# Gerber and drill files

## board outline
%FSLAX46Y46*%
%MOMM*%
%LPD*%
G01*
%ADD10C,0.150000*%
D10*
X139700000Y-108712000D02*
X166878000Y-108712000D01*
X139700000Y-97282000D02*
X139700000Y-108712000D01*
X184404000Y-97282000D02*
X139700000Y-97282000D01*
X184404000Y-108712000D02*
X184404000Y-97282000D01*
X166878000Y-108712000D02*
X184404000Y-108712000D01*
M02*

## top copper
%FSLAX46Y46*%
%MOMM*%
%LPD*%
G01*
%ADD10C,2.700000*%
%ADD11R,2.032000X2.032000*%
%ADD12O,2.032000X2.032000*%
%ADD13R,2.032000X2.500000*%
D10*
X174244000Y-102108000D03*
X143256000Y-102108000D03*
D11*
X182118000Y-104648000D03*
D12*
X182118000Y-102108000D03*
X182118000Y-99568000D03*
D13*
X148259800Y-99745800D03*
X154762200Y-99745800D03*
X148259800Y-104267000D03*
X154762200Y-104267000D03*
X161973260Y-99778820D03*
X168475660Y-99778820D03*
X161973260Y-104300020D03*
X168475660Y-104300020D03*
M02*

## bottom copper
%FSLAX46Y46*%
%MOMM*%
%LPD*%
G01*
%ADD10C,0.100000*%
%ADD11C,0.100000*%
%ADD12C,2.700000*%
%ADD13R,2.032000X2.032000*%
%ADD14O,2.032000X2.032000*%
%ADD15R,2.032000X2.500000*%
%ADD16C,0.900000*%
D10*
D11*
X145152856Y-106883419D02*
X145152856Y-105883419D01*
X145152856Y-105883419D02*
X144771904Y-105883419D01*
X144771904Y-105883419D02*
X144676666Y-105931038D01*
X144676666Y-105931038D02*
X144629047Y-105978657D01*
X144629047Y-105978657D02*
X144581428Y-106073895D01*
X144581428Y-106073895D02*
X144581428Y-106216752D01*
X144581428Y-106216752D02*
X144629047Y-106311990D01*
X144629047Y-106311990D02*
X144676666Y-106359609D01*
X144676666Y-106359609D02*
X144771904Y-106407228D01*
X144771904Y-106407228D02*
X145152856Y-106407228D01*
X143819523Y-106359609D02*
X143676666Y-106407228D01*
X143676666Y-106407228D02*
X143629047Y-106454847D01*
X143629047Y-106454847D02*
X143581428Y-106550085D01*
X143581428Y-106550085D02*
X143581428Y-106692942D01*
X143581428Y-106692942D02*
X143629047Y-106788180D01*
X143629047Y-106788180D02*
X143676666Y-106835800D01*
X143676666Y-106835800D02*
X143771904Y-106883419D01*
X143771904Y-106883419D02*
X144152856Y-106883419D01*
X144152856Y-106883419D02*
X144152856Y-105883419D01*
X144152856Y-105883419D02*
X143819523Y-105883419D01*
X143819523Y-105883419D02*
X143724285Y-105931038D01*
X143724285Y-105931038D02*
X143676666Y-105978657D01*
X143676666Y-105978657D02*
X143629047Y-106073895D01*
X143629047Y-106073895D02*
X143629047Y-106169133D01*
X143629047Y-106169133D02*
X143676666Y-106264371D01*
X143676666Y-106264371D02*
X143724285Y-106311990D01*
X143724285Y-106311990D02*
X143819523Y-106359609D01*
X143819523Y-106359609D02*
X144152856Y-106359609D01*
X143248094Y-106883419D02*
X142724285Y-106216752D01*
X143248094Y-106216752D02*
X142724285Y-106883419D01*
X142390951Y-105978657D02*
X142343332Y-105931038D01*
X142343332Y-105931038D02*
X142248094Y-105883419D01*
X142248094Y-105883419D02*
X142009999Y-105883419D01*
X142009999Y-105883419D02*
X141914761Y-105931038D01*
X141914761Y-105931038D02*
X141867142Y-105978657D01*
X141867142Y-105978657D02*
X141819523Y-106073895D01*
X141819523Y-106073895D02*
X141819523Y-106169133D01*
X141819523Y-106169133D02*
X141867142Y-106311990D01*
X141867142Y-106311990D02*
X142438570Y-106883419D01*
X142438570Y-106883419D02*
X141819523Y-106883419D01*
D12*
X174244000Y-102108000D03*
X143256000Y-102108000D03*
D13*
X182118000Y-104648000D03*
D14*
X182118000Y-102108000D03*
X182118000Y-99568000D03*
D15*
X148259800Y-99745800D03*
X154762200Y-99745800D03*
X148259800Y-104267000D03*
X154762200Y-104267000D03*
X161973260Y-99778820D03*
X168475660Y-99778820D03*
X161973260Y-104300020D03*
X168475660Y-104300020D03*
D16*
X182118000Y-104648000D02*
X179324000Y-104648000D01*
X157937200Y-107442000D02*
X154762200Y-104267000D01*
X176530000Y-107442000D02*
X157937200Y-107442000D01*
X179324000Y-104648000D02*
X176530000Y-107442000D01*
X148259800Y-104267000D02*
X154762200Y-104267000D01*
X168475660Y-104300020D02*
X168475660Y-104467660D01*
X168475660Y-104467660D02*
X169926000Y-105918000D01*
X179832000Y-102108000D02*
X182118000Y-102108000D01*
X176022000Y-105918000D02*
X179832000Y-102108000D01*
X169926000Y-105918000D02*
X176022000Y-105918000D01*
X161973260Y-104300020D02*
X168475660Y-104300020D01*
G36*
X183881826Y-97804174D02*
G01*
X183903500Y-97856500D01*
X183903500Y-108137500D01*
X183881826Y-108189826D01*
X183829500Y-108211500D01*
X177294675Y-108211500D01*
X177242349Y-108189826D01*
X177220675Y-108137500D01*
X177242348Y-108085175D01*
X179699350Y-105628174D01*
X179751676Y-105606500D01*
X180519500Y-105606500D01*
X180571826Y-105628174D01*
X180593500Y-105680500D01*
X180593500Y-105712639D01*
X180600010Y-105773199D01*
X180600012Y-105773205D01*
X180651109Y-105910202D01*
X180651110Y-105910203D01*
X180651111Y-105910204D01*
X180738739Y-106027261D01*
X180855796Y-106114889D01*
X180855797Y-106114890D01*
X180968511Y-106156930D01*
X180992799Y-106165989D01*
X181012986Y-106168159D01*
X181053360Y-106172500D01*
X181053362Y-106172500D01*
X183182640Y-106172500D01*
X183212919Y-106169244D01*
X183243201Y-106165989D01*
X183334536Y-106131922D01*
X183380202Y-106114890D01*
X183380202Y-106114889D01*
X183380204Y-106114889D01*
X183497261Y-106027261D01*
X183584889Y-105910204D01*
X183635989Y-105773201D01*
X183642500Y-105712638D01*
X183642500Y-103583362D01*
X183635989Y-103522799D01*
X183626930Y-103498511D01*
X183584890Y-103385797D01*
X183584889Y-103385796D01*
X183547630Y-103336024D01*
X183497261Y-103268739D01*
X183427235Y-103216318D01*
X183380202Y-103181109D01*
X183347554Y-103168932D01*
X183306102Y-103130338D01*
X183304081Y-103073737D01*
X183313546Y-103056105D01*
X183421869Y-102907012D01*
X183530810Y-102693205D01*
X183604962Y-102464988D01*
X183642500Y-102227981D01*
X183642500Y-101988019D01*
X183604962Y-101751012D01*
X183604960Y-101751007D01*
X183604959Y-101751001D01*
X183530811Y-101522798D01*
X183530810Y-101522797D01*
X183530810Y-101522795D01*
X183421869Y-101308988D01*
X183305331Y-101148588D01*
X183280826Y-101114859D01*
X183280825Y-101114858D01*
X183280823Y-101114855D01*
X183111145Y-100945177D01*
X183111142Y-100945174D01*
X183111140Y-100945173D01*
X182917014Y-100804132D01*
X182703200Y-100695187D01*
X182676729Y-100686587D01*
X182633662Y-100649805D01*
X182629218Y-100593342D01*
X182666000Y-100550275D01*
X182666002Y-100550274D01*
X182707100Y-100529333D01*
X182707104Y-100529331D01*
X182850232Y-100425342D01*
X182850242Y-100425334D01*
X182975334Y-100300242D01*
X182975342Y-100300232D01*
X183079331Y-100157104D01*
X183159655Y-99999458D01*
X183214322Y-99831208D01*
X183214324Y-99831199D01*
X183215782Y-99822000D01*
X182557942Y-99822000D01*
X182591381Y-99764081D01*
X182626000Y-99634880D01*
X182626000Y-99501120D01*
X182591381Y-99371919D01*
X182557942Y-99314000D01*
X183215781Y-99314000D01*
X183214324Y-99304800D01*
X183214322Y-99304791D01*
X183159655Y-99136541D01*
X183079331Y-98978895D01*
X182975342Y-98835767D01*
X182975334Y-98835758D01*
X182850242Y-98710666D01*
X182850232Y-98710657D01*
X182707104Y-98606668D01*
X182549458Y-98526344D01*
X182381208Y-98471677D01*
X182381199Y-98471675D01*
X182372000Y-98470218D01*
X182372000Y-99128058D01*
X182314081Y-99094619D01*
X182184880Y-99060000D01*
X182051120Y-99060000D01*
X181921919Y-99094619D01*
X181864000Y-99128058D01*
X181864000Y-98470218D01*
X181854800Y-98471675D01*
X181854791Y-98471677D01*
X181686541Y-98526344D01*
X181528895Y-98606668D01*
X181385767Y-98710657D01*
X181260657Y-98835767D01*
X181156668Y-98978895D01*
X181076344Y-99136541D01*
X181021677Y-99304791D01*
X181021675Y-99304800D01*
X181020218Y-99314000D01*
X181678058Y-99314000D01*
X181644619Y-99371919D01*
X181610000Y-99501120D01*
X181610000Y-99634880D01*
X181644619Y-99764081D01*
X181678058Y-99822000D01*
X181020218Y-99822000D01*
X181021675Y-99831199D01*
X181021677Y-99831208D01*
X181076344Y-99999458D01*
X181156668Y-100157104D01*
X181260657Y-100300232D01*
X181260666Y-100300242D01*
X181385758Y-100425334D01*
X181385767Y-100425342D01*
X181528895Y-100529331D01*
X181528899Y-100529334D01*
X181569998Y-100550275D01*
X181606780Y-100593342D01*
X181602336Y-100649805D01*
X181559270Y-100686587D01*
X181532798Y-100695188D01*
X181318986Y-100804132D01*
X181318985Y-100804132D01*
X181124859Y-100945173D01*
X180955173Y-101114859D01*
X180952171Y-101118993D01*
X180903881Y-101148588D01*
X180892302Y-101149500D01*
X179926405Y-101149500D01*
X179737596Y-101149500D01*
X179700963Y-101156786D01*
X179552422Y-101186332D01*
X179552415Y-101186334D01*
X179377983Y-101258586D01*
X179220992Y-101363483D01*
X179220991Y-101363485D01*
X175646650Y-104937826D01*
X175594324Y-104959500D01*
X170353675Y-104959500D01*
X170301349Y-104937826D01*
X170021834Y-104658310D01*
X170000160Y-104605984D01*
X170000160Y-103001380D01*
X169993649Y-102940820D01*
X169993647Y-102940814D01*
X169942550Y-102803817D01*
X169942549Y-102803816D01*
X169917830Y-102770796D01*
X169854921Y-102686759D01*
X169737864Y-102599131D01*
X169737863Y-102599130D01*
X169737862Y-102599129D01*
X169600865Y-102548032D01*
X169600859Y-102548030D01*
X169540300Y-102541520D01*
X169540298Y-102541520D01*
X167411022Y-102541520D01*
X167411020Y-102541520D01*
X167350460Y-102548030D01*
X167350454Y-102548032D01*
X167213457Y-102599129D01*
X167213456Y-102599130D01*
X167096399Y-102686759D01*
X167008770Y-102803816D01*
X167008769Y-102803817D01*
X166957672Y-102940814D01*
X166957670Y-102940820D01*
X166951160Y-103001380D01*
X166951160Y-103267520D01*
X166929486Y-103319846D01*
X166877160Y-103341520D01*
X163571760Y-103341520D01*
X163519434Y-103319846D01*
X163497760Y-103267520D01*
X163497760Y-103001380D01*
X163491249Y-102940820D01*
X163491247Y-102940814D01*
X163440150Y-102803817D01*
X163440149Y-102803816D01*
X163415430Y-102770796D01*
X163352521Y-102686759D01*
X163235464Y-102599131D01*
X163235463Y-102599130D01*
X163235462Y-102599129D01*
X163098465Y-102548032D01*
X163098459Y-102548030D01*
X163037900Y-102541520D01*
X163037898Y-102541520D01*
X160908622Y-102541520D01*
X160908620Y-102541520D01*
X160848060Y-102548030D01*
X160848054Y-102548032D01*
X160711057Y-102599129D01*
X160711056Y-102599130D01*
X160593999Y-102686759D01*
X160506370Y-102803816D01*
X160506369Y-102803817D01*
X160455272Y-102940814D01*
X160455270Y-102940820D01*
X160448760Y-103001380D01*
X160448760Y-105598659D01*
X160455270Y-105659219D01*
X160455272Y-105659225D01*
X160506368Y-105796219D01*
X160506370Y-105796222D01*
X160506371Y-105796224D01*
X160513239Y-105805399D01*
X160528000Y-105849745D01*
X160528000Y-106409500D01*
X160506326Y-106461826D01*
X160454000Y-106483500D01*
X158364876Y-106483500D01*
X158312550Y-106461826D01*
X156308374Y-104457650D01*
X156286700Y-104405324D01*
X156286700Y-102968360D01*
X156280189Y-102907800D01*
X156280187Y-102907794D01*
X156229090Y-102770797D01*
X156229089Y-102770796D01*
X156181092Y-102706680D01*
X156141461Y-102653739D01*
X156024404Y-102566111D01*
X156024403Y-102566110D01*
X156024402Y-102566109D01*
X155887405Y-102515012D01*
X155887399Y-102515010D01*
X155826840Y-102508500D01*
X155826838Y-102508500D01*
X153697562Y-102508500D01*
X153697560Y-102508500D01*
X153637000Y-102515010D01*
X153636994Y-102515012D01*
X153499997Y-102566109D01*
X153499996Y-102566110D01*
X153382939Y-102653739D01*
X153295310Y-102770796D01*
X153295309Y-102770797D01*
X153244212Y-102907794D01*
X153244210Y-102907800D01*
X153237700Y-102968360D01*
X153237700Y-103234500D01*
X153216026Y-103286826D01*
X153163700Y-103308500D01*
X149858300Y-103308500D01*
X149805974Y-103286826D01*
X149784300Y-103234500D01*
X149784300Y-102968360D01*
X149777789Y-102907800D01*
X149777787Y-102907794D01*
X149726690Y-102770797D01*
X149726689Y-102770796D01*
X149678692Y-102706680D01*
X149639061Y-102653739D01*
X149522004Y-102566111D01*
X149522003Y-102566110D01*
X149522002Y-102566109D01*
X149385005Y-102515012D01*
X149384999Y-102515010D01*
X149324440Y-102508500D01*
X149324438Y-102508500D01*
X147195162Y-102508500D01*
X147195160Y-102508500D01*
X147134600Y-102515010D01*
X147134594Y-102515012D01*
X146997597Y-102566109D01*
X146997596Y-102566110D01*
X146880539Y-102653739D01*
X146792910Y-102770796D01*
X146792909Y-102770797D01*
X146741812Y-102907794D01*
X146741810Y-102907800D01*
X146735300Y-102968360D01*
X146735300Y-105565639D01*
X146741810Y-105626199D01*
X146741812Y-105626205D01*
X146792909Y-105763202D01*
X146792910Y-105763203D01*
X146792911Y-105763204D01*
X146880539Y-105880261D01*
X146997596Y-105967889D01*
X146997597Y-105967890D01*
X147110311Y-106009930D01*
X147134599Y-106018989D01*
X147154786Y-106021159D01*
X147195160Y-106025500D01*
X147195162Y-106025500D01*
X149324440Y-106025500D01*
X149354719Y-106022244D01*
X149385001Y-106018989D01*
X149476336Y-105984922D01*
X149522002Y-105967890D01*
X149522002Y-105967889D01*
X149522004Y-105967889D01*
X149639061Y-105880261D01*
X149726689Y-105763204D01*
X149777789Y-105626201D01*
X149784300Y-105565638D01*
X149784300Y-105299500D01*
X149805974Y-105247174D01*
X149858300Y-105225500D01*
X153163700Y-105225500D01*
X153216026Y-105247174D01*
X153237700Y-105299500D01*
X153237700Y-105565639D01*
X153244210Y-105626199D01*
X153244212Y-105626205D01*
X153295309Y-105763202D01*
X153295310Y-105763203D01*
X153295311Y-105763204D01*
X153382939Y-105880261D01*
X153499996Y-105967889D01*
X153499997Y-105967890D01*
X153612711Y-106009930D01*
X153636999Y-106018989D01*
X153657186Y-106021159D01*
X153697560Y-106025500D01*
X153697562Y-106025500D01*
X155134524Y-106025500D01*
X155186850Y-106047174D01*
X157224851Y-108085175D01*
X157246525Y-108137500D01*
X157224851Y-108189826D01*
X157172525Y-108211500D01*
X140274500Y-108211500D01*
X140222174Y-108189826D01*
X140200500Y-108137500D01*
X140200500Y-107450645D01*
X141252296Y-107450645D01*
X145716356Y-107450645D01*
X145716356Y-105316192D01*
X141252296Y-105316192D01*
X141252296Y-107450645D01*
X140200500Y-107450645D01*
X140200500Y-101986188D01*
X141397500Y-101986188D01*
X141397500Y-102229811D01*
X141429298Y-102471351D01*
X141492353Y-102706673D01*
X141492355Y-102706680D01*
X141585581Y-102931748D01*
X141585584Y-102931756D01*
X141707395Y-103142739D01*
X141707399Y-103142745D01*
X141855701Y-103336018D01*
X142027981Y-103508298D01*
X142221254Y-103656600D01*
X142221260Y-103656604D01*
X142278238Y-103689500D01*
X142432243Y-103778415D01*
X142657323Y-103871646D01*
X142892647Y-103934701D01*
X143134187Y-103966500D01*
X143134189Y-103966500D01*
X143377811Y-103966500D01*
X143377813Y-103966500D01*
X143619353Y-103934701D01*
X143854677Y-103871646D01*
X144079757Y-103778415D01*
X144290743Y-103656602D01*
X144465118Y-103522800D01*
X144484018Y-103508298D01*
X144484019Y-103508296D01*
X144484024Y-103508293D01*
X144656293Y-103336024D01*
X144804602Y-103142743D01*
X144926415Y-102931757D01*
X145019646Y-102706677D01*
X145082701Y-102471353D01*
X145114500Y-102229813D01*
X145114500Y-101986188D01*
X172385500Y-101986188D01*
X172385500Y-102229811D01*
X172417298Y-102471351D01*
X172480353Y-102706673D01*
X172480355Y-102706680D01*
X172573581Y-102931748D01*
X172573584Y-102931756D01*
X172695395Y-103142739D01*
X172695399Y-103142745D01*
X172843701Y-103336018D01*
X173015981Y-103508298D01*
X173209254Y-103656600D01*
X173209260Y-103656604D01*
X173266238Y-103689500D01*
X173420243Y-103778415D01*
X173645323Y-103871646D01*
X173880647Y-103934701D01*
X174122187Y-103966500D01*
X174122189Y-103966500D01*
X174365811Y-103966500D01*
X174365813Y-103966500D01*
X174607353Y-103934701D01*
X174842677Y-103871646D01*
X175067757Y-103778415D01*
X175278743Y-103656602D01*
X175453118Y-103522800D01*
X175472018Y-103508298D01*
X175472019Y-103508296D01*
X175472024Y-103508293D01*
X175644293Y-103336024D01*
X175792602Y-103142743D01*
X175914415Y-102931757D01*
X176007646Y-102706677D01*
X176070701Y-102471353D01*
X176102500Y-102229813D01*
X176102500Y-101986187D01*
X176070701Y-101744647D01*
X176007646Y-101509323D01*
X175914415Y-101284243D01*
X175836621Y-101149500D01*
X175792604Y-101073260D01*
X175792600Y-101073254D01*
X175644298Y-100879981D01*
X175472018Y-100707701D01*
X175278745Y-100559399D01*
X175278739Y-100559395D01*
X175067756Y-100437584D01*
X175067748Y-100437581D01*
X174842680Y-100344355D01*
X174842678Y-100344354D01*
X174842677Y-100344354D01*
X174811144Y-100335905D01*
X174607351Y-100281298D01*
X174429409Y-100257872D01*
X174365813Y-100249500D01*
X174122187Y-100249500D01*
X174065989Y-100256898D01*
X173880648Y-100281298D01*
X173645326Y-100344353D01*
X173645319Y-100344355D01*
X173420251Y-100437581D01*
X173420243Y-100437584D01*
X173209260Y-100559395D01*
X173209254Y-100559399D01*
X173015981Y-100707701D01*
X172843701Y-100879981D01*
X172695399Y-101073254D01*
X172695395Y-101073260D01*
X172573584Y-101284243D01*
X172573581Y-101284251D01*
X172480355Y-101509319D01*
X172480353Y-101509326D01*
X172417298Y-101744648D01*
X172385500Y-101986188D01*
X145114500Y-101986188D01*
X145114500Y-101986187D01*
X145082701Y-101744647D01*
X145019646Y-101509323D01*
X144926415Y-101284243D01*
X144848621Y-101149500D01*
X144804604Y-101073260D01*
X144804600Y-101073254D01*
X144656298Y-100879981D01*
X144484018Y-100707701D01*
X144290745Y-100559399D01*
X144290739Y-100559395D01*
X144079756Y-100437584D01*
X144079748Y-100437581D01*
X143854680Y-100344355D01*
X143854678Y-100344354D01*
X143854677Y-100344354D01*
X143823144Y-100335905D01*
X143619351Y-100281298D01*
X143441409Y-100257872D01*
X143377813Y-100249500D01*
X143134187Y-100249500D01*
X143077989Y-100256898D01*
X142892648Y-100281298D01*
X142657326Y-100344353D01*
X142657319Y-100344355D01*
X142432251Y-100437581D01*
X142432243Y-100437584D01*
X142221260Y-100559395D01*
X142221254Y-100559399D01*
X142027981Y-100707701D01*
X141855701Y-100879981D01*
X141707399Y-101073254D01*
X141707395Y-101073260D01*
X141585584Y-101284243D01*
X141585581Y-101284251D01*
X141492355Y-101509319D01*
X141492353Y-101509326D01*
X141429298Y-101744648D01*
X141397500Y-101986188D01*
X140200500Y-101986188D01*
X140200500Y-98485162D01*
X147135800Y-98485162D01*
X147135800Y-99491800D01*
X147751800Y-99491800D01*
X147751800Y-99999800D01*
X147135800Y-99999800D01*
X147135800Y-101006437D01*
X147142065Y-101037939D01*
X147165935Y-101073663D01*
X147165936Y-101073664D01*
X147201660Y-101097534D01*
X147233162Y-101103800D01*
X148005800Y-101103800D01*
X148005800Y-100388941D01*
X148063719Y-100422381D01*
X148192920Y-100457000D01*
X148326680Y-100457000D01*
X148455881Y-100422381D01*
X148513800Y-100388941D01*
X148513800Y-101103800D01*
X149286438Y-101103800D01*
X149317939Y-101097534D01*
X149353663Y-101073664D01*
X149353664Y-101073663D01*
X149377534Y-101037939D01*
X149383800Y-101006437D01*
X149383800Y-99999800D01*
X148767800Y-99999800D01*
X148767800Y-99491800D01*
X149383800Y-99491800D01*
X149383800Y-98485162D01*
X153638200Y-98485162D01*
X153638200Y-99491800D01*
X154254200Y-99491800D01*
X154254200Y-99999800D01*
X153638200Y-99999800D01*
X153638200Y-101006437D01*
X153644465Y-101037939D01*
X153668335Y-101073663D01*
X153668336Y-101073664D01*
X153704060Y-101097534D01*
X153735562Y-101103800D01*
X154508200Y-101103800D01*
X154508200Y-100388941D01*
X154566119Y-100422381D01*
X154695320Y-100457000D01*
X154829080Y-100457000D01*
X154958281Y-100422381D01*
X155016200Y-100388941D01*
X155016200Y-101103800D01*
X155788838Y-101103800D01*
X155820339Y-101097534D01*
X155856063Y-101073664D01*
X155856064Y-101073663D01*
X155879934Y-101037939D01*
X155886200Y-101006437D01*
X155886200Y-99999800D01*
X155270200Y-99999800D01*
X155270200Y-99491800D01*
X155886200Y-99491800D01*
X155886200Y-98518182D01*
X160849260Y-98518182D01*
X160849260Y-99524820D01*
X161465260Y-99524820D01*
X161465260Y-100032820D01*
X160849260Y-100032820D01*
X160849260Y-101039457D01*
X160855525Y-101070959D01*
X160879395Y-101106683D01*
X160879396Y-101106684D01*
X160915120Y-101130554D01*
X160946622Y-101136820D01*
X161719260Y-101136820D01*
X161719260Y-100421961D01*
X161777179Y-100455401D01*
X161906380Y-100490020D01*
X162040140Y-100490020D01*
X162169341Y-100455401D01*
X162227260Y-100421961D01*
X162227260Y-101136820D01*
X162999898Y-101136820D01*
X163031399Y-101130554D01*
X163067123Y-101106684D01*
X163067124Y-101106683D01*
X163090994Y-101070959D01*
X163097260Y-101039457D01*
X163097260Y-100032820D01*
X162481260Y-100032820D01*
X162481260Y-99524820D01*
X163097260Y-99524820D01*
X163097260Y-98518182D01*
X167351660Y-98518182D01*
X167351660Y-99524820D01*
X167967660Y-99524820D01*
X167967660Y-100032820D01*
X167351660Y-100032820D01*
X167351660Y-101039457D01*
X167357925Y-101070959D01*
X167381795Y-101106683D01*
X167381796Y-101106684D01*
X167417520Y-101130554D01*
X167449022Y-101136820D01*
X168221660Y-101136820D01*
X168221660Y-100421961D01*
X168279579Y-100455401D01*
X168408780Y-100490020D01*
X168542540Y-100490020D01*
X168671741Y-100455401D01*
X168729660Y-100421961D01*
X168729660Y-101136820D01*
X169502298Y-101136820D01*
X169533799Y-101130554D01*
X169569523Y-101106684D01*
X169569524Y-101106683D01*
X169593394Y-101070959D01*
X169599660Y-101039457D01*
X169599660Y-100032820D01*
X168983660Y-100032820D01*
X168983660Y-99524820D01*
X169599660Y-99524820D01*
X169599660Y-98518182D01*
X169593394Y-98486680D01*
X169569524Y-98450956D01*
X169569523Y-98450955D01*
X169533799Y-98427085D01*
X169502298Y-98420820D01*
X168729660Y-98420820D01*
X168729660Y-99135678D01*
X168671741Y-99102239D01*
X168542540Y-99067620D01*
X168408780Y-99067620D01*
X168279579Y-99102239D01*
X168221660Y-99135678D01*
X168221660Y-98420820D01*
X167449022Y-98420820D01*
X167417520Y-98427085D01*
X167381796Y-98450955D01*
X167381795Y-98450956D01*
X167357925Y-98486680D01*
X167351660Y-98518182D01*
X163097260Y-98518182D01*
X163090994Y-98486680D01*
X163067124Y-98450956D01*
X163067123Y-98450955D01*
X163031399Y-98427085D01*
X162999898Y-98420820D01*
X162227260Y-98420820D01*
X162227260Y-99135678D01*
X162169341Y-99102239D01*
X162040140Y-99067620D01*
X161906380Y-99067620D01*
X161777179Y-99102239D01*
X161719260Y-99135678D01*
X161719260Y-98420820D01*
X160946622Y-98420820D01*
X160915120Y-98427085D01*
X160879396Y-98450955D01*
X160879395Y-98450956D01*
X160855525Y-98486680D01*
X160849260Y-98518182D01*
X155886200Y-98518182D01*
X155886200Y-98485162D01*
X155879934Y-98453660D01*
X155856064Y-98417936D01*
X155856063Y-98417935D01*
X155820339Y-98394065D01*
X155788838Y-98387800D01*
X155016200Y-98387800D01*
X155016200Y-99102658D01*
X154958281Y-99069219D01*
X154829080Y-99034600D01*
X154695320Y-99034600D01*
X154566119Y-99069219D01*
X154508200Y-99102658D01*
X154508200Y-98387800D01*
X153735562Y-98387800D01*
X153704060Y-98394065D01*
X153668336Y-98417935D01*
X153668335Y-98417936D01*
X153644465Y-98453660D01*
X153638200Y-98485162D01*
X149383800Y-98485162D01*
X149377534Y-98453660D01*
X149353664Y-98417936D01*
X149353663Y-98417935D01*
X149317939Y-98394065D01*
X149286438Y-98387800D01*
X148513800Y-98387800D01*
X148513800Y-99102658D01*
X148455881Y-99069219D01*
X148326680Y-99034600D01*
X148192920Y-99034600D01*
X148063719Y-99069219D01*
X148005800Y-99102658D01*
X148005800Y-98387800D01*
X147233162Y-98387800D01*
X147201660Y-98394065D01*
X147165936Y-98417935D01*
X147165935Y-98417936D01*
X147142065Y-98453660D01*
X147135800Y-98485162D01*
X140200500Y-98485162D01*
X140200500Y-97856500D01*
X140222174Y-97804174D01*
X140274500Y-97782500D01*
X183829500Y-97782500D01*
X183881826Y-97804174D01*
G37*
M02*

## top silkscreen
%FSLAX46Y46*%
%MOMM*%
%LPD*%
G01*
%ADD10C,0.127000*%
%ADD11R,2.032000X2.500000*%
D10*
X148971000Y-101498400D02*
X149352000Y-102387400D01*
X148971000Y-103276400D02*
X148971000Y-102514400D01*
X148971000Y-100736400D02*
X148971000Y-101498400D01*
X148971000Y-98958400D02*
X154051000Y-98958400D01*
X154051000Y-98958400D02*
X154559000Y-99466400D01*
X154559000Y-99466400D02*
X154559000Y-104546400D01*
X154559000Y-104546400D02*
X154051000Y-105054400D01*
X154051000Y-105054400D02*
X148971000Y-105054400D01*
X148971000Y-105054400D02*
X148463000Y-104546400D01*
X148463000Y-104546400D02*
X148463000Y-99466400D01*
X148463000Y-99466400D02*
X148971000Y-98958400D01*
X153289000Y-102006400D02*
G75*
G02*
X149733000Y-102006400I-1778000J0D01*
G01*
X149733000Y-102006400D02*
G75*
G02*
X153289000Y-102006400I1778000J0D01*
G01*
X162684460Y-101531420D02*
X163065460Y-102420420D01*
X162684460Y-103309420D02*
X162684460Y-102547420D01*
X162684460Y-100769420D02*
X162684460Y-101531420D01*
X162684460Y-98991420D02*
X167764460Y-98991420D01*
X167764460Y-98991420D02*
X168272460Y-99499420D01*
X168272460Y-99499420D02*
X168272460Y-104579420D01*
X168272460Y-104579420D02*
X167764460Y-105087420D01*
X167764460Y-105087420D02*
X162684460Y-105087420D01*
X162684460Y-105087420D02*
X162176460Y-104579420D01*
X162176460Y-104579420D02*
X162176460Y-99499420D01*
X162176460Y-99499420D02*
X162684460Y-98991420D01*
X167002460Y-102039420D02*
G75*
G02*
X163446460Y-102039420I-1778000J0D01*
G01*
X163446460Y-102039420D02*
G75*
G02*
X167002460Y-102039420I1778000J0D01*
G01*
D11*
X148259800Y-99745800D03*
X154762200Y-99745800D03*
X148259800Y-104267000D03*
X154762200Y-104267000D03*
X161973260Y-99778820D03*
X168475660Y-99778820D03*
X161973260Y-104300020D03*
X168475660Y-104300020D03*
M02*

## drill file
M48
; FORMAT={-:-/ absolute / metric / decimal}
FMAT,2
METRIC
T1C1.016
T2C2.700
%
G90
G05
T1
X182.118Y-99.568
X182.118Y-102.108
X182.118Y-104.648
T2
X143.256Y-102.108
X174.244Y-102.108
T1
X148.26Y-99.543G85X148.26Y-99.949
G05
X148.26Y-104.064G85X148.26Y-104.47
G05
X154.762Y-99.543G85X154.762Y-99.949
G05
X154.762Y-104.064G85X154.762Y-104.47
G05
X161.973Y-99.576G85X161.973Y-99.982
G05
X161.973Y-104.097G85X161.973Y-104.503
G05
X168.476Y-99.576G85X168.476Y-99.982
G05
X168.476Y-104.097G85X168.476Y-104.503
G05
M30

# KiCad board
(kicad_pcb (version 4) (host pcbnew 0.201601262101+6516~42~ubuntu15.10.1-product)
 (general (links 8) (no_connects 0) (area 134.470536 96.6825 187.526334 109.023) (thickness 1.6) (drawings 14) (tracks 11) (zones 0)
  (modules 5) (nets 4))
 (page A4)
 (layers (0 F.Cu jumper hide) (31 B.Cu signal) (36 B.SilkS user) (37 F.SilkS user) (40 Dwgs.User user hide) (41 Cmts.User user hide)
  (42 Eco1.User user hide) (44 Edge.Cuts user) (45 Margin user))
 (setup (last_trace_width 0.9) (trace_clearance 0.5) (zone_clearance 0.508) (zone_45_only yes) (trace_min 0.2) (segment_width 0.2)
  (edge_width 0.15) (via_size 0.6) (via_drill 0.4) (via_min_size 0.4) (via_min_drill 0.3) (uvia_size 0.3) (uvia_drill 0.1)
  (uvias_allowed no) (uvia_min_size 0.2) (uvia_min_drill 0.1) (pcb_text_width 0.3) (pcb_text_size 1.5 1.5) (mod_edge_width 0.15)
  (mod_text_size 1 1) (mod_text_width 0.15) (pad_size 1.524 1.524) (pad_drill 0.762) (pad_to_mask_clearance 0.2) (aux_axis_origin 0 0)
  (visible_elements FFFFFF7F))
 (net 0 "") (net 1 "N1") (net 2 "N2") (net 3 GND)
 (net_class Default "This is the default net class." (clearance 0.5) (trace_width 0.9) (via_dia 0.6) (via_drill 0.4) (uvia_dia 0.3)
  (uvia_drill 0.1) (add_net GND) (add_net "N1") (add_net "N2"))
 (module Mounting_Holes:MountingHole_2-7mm (layer F.Cu) (at 174.244 102.108)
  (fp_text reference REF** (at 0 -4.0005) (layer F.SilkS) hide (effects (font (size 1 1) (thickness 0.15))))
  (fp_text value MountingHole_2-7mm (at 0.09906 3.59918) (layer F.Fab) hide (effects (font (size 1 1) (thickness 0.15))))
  (pad 1 thru_hole circle (at 0 0) (size 2.7 2.7) (drill 2.7) (layers)))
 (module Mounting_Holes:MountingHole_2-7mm (layer F.Cu) (at 143.256 102.108)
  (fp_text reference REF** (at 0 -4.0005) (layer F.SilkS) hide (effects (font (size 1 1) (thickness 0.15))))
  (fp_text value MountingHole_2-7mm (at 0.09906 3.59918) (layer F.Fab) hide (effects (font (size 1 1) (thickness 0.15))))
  (pad 1 thru_hole circle (at 0 0) (size 2.7 2.7) (drill 2.7) (layers)))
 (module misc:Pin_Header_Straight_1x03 (layer B.Cu) (at 182.118 104.648)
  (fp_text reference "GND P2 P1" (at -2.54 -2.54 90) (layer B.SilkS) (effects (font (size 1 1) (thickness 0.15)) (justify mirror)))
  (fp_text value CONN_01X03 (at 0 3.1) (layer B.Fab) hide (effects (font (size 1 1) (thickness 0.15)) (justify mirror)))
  (pad 1 thru_hole rect (at 0 0) (size 2.032 2.032) (drill 1.016) (layers *.Cu *.Mask B.SilkS) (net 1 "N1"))
  (pad 2 thru_hole oval (at 0 -2.54) (size 2.032 2.032) (drill 1.016) (layers *.Cu *.Mask B.SilkS) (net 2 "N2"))
  (pad 3 thru_hole oval (at 0 -5.08) (size 2.032 2.032) (drill 1.016) (layers *.Cu *.Mask B.SilkS) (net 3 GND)))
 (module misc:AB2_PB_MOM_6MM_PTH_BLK (layer F.Cu) (at 151.511 102.0064)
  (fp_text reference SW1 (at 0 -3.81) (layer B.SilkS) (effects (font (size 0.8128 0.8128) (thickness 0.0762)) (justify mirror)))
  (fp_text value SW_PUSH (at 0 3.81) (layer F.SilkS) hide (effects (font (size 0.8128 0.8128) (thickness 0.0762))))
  (fp_line (start -2.54 -0.508) (end -2.159 0.381) (layer F.SilkS) (width 0.127))
  (fp_line (start -2.54 1.27) (end -2.54 0.508) (layer F.SilkS) (width 0.127))
  (fp_line (start -2.54 -1.27) (end -2.54 -0.508) (layer F.SilkS) (width 0.127))
  (fp_line (start -2.54 -3.048) (end 2.54 -3.048) (layer F.SilkS) (width 0.127))
  (fp_line (start 2.54 -3.048) (end 3.048 -2.54) (layer F.SilkS) (width 0.127))
  (fp_line (start 3.048 -2.54) (end 3.048 2.54) (layer F.SilkS) (width 0.127))
  (fp_line (start 3.048 2.54) (end 2.54 3.048) (layer F.SilkS) (width 0.127))
  (fp_line (start 2.54 3.048) (end -2.54 3.048) (layer F.SilkS) (width 0.127))
  (fp_line (start -2.54 3.048) (end -3.048 2.54) (layer F.SilkS) (width 0.127))
  (fp_line (start -3.048 2.54) (end -3.048 -2.54) (layer F.SilkS) (width 0.127))
  (fp_line (start -3.048 -2.54) (end -2.54 -3.048) (layer F.SilkS) (width 0.127))
  (fp_circle (center 0 0) (end 0 -1.778) (layer F.SilkS) (width 0.127))
  (pad 1 thru_hole rect (at -3.2512 -2.2606) (size 2.032 2.5) (drill oval 1.016 1.4224) (layers *.Cu *.Mask F.SilkS) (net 3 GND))
  (pad 1 thru_hole rect (at 3.2512 -2.2606) (size 2.032 2.5) (drill oval 1.016 1.4224) (layers *.Cu *.Mask F.SilkS) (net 3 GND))
  (pad 2 thru_hole rect (at -3.2512 2.2606) (size 2.032 2.5) (drill oval 1.016 1.4224) (layers *.Cu *.Mask F.SilkS) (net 1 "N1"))
  (pad 2 thru_hole rect (at 3.2512 2.2606) (size 2.032 2.5) (drill oval 1.016 1.4224) (layers *.Cu *.Mask F.SilkS) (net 1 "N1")))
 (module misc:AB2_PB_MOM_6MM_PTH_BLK (layer F.Cu) (at 165.22446 102.03942)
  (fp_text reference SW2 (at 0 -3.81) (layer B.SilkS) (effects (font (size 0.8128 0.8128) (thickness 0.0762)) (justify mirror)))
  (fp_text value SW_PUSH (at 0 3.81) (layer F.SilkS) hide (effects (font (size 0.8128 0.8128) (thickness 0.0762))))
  (fp_line (start -2.54 -0.508) (end -2.159 0.381) (layer F.SilkS) (width 0.127))
  (fp_line (start -2.54 1.27) (end -2.54 0.508) (layer F.SilkS) (width 0.127))
  (fp_line (start -2.54 -1.27) (end -2.54 -0.508) (layer F.SilkS) (width 0.127))
  (fp_line (start -2.54 -3.048) (end 2.54 -3.048) (layer F.SilkS) (width 0.127))
  (fp_line (start 2.54 -3.048) (end 3.048 -2.54) (layer F.SilkS) (width 0.127))
  (fp_line (start 3.048 -2.54) (end 3.048 2.54) (layer F.SilkS) (width 0.127))
  (fp_line (start 3.048 2.54) (end 2.54 3.048) (layer F.SilkS) (width 0.127))
  (fp_line (start 2.54 3.048) (end -2.54 3.048) (layer F.SilkS) (width 0.127))
  (fp_line (start -2.54 3.048) (end -3.048 2.54) (layer F.SilkS) (width 0.127))
  (fp_line (start -3.048 2.54) (end -3.048 -2.54) (layer F.SilkS) (width 0.127))
  (fp_line (start -3.048 -2.54) (end -2.54 -3.048) (layer F.SilkS) (width 0.127))
  (fp_circle (center 0 0) (end 0 -1.778) (layer F.SilkS) (width 0.127))
  (pad 1 thru_hole rect (at -3.2512 -2.2606) (size 2.032 2.5) (drill oval 1.016 1.4224) (layers *.Cu *.Mask F.SilkS) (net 3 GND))
  (pad 1 thru_hole rect (at 3.2512 -2.2606) (size 2.032 2.5) (drill oval 1.016 1.4224) (layers *.Cu *.Mask F.SilkS) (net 3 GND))
  (pad 2 thru_hole rect (at -3.2512 2.2606) (size 2.032 2.5) (drill oval 1.016 1.4224) (layers *.Cu *.Mask F.SilkS) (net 2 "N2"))
  (pad 2 thru_hole rect (at 3.2512 2.2606) (size 2.032 2.5) (drill oval 1.016 1.4224) (layers *.Cu *.Mask F.SilkS) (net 2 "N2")))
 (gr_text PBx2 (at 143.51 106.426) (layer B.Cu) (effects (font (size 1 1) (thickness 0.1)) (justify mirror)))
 (gr_line (start 139.7 108.712) (end 166.878 108.712) (angle 90) (layer Edge.Cuts) (width 0.15))
 (gr_line (start 139.7 97.282) (end 139.7 108.712) (angle 90) (layer Edge.Cuts) (width 0.15))
 (gr_line (start 184.404 97.282) (end 139.7 97.282) (angle 90) (layer Edge.Cuts) (width 0.15))
 (gr_line (start 184.404 108.712) (end 184.404 97.282) (angle 90) (layer Edge.Cuts) (width 0.15))
 (gr_line (start 166.878 108.712) (end 184.404 108.712) (angle 90) (layer Edge.Cuts) (width 0.15))
 (segment (start 182.118 104.648) (end 179.324 104.648) (width 0.9) (layer B.Cu) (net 1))
 (segment (start 157.9372 107.442) (end 154.7622 104.267) (width 0.9) (layer B.Cu) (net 1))
 (segment (start 176.53 107.442) (end 157.9372 107.442) (width 0.9) (layer B.Cu) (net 1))
 (segment (start 179.324 104.648) (end 176.53 107.442) (width 0.9) (layer B.Cu) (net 1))
 (segment (start 148.2598 104.267) (end 154.7622 104.267) (width 0.9) (layer B.Cu) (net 1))
 (segment (start 168.47566 104.30002) (end 168.47566 104.46766) (width 0.9) (layer B.Cu) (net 2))
 (segment (start 168.47566 104.46766) (end 169.926 105.918) (width 0.9) (layer B.Cu) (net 2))
 (segment (start 179.832 102.108) (end 182.118 102.108) (width 0.9) (layer B.Cu) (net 2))
 (segment (start 176.022 105.918) (end 179.832 102.108) (width 0.9) (layer B.Cu) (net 2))
 (segment (start 169.926 105.918) (end 176.022 105.918) (width 0.9) (layer B.Cu) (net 2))
 (segment (start 161.97326 104.30002) (end 168.47566 104.30002) (width 0.9) (layer B.Cu) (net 2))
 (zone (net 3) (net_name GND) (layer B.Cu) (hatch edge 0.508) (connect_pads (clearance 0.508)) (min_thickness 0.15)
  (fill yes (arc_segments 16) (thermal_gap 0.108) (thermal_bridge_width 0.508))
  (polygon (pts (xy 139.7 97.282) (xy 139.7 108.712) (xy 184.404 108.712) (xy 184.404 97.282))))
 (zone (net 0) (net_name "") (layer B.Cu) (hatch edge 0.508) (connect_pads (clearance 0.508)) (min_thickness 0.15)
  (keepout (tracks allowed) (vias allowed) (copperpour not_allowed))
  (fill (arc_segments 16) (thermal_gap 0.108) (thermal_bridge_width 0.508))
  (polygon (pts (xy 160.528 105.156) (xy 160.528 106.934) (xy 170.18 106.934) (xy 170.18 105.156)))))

